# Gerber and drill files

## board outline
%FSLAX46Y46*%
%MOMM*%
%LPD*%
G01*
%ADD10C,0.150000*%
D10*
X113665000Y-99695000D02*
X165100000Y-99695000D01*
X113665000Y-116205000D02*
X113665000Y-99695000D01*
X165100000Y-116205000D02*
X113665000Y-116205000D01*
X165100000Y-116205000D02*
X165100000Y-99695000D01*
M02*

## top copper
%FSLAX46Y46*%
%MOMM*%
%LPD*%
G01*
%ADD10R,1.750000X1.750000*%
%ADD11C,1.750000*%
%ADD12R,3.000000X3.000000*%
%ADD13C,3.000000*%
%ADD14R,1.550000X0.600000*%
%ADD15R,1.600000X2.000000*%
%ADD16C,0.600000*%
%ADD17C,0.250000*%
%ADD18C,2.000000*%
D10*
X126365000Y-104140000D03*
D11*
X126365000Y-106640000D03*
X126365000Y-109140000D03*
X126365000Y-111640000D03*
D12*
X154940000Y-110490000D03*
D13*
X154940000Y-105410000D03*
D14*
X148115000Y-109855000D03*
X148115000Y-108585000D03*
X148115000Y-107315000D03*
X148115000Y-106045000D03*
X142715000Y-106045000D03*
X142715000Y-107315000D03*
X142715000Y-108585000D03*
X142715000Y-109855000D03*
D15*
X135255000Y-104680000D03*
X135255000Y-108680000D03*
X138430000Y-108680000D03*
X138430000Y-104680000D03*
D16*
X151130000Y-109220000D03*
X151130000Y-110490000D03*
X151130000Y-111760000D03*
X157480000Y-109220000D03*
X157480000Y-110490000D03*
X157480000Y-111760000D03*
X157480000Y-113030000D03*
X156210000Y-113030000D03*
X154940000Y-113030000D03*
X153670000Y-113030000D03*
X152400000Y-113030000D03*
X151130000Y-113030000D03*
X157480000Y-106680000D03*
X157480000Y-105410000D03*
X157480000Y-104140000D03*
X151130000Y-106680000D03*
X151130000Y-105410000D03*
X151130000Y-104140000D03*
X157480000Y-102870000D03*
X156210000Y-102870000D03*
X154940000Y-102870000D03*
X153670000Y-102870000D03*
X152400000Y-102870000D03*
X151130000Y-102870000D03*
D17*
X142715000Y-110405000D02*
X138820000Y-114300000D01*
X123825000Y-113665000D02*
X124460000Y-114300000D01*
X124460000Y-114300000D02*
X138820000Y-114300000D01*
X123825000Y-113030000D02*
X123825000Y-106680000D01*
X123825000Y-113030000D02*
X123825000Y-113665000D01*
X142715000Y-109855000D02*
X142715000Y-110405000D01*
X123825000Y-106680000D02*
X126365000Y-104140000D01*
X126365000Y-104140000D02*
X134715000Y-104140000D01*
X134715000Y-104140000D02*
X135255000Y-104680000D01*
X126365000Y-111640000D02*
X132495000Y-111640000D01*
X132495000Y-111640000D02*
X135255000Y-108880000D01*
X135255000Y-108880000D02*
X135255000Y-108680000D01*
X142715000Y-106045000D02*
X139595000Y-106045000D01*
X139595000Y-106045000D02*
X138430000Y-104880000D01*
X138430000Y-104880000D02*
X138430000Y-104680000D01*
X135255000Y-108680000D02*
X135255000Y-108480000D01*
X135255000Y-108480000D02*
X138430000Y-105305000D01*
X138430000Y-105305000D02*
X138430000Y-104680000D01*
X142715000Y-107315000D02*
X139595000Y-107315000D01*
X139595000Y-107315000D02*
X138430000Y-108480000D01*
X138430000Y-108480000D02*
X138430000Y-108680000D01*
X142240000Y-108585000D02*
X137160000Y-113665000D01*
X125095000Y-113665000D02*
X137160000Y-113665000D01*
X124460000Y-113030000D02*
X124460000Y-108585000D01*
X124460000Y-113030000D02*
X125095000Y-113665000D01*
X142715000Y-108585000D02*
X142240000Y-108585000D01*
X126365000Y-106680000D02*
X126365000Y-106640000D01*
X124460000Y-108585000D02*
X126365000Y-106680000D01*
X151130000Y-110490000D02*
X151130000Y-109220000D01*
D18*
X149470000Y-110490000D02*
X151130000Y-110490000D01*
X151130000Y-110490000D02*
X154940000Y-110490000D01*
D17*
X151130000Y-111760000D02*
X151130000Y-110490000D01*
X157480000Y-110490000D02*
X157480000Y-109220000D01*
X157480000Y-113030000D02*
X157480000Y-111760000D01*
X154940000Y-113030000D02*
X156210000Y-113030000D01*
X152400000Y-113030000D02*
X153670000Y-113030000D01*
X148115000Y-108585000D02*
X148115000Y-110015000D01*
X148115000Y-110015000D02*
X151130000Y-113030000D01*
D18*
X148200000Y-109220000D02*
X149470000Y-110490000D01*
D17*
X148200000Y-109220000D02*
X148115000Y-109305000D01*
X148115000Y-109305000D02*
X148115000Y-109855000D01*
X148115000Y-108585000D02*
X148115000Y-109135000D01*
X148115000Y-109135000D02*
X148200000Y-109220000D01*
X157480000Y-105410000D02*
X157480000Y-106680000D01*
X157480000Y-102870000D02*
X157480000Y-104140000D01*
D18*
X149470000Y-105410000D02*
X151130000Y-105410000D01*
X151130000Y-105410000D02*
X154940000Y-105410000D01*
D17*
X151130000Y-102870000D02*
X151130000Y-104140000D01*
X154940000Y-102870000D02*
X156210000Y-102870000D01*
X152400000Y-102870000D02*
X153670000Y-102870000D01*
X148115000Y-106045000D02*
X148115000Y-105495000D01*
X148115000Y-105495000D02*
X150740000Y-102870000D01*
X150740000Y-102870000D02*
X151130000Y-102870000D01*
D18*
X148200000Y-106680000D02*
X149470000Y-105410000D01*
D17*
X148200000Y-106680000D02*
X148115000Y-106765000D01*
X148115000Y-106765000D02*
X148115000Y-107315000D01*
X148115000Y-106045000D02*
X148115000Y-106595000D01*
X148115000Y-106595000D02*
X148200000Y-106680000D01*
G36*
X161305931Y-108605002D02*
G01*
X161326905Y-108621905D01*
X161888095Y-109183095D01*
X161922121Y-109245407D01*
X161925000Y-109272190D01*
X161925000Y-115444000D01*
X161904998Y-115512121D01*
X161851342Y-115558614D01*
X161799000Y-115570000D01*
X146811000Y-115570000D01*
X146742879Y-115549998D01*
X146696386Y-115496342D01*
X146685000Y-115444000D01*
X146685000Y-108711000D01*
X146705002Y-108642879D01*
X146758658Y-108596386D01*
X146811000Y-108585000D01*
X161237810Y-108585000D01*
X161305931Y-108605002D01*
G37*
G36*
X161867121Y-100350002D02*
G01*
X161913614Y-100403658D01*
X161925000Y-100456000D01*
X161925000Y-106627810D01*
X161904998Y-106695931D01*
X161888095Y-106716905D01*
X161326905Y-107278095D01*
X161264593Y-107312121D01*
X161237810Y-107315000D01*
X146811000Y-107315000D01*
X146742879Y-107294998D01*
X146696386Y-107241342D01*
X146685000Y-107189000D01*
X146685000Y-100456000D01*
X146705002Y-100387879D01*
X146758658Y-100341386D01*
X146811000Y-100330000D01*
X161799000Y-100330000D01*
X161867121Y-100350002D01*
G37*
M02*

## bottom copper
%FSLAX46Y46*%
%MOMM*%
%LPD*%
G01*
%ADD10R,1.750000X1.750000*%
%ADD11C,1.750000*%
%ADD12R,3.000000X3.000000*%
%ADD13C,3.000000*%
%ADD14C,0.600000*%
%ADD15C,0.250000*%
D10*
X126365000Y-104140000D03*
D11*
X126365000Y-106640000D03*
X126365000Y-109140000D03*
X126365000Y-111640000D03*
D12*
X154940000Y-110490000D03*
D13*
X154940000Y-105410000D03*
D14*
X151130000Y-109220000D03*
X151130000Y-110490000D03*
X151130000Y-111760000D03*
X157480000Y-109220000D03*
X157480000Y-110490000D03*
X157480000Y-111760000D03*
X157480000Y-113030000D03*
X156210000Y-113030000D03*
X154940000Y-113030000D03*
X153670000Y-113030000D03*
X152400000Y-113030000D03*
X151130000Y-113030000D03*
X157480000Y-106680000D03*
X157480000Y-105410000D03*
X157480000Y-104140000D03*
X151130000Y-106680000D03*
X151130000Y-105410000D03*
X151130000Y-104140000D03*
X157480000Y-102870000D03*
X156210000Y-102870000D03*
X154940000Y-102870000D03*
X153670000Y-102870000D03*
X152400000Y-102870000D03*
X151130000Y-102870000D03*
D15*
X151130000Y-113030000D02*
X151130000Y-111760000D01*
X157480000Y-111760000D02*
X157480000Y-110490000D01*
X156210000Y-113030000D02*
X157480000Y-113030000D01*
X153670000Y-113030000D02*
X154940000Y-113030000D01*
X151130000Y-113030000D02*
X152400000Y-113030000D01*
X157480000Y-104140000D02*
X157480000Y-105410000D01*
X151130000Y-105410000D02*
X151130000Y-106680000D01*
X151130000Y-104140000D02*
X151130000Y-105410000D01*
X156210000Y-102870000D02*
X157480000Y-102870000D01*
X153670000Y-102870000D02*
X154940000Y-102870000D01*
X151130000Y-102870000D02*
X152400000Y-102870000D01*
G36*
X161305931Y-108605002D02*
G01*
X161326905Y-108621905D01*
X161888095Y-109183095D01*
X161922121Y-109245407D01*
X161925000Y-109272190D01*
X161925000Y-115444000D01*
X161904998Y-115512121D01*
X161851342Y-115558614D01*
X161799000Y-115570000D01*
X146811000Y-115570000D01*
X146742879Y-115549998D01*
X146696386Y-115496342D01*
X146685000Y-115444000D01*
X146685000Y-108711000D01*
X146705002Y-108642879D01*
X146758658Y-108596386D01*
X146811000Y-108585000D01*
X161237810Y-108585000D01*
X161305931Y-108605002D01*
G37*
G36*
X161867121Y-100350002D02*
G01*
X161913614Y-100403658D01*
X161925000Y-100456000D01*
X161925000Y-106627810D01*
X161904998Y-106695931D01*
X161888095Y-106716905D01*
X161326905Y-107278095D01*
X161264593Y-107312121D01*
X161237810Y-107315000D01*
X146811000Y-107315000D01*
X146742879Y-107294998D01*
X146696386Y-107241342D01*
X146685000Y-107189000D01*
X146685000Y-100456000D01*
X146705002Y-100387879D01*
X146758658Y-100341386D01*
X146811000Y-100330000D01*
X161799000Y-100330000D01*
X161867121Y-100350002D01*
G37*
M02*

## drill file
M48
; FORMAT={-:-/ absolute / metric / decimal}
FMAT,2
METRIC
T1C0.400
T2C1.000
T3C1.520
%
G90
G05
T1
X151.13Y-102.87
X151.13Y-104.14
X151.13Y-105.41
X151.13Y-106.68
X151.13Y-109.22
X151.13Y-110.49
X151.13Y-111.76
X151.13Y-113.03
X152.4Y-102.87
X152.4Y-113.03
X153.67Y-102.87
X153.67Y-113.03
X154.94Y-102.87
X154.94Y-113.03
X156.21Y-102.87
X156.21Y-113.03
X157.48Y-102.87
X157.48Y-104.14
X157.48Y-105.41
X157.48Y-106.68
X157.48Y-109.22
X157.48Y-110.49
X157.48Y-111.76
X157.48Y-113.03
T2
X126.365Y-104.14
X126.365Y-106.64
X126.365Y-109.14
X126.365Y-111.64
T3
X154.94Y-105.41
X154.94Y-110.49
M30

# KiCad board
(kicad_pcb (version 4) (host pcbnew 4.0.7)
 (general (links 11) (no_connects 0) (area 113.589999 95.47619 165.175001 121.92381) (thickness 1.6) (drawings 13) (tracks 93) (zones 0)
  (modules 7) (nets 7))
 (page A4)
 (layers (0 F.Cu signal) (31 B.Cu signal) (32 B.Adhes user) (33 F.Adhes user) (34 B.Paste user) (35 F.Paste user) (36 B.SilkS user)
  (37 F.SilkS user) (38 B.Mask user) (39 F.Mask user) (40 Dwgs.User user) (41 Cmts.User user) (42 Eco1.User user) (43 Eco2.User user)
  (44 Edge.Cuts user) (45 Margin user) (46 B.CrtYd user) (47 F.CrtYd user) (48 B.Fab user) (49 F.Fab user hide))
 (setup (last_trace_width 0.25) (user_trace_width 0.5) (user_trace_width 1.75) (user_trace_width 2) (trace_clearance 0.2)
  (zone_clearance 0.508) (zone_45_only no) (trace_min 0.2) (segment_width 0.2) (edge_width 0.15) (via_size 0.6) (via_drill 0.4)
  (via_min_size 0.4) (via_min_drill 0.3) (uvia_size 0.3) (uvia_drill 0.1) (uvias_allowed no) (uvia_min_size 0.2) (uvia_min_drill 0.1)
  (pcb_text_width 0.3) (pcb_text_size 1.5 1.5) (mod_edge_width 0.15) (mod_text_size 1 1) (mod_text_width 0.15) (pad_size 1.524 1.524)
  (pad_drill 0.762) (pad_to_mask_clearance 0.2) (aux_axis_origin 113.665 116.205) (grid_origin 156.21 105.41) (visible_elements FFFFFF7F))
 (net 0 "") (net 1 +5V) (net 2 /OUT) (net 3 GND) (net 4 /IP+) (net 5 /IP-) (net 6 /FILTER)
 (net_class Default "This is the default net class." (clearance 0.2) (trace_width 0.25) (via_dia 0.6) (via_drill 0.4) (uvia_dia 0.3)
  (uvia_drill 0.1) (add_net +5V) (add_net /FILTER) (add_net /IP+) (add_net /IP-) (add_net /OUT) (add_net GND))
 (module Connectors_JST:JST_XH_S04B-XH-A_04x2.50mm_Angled (layer F.Cu) (at 126.365 104.14 270)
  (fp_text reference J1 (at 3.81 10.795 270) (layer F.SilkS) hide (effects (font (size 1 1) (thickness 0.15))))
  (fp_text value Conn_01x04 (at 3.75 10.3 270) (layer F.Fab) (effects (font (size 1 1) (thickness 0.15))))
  (pad 1 thru_hole rect (at 0 0 270) (size 1.75 1.75) (drill 1) (layers *.Cu *.Mask F.SilkS) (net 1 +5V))
  (pad 2 thru_hole circle (at 2.5 0 270) (size 1.75 1.75) (drill 1) (layers *.Cu *.Mask F.SilkS) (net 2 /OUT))
  (pad 3 thru_hole circle (at 5 0 270) (size 1.75 1.75) (drill 1) (layers *.Cu *.Mask F.SilkS))
  (pad 4 thru_hole circle (at 7.5 0 270) (size 1.75 1.75) (drill 1) (layers *.Cu *.Mask F.SilkS) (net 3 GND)))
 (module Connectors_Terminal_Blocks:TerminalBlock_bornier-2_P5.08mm (layer F.Cu) (at 154.94 110.49 90)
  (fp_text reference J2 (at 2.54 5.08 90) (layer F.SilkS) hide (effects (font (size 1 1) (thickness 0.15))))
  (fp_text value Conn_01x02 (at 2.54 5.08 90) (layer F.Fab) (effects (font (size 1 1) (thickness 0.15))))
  (pad 1 thru_hole rect (at 0 0 90) (size 3 3) (drill 1.52) (layers *.Cu *.Mask) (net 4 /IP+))
  (pad 2 thru_hole circle (at 5.08 0 90) (size 3 3) (drill 1.52) (layers *.Cu *.Mask) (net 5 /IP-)))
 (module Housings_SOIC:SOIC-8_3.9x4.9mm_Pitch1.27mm (layer F.Cu) (at 145.415 107.95 180)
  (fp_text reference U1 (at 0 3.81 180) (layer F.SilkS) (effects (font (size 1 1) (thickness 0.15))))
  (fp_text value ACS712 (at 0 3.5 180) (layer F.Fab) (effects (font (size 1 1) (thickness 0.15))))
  (pad 1 smd rect (at -2.7 -1.905 180) (size 1.55 0.6) (layers F.Cu F.Paste F.Mask) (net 4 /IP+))
  (pad 2 smd rect (at -2.7 -0.635 180) (size 1.55 0.6) (layers F.Cu F.Paste F.Mask) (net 4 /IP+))
  (pad 3 smd rect (at -2.7 0.635 180) (size 1.55 0.6) (layers F.Cu F.Paste F.Mask) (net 5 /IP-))
  (pad 4 smd rect (at -2.7 1.905 180) (size 1.55 0.6) (layers F.Cu F.Paste F.Mask) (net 5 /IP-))
  (pad 5 smd rect (at 2.7 1.905 180) (size 1.55 0.6) (layers F.Cu F.Paste F.Mask) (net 3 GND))
  (pad 6 smd rect (at 2.7 0.635 180) (size 1.55 0.6) (layers F.Cu F.Paste F.Mask) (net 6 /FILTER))
  (pad 7 smd rect (at 2.7 -0.635 180) (size 1.55 0.6) (layers F.Cu F.Paste F.Mask) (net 2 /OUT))
  (pad 8 smd rect (at 2.7 -1.905 180) (size 1.55 0.6) (layers F.Cu F.Paste F.Mask) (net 1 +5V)))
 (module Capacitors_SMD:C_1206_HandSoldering (layer F.Cu) (at 135.255 106.68 270)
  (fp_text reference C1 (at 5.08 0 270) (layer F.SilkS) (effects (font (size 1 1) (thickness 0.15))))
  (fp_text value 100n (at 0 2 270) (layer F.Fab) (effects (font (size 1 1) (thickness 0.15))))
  (pad 1 smd rect (at -2 0 270) (size 2 1.6) (layers F.Cu F.Paste F.Mask) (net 1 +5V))
  (pad 2 smd rect (at 2 0 270) (size 2 1.6) (layers F.Cu F.Paste F.Mask) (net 3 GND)))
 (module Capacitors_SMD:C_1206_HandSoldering (layer F.Cu) (at 138.43 106.68 90)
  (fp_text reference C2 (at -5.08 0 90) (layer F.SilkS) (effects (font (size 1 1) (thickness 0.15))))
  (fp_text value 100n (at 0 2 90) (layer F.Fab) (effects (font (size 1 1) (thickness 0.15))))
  (pad 1 smd rect (at -2 0 90) (size 2 1.6) (layers F.Cu F.Paste F.Mask) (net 6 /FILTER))
  (pad 2 smd rect (at 2 0 90) (size 2 1.6) (layers F.Cu F.Paste F.Mask) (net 3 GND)))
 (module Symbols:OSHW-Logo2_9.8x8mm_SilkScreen (layer B.Cu) (at 120.015 107.95 270)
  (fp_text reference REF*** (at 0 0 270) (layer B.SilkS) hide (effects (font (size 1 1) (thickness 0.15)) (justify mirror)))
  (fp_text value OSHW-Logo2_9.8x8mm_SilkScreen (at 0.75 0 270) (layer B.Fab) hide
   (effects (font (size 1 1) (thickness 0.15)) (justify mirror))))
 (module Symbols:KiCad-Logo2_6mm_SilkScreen (layer B.Cu) (at 160.655 107.95 270)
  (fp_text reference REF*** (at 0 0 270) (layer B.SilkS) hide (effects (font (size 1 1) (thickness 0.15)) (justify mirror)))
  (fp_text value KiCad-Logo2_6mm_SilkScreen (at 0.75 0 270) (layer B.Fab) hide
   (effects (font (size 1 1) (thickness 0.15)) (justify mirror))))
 (gr_line (start 113.665 99.695) (end 165.1 99.695) (layer Edge.Cuts) (width 0.15))
 (gr_line (start 113.665 116.205) (end 113.665 99.695) (layer Edge.Cuts) (width 0.15))
 (gr_line (start 165.1 116.205) (end 113.665 116.205) (layer Edge.Cuts) (width 0.15))
 (gr_line (start 165.1 116.205) (end 165.1 99.695) (layer Edge.Cuts) (width 0.15))
 (segment (start 142.715 110.405) (end 138.82 114.3) (width 0.25) (layer F.Cu) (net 1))
 (segment (start 123.825 113.665) (end 124.46 114.3) (width 0.25) (layer F.Cu) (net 1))
 (segment (start 124.46 114.3) (end 138.82 114.3) (width 0.25) (layer F.Cu) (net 1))
 (segment (start 123.825 113.03) (end 123.825 106.68) (width 0.25) (layer F.Cu) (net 1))
 (segment (start 123.825 113.03) (end 123.825 113.665) (width 0.25) (layer F.Cu) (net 1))
 (segment (start 142.715 109.855) (end 142.715 110.405) (width 0.25) (layer F.Cu) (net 1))
 (segment (start 123.825 106.68) (end 126.365 104.14) (width 0.25) (layer F.Cu) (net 1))
 (segment (start 126.365 104.14) (end 134.715 104.14) (width 0.25) (layer F.Cu) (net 1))
 (segment (start 134.715 104.14) (end 135.255 104.68) (width 0.25) (layer F.Cu) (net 1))
 (segment (start 126.365 111.64) (end 132.495 111.64) (width 0.25) (layer F.Cu) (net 3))
 (segment (start 132.495 111.64) (end 135.255 108.88) (width 0.25) (layer F.Cu) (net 3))
 (segment (start 135.255 108.88) (end 135.255 108.68) (width 0.25) (layer F.Cu) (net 3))
 (segment (start 142.715 106.045) (end 139.595 106.045) (width 0.25) (layer F.Cu) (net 3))
 (segment (start 139.595 106.045) (end 138.43 104.88) (width 0.25) (layer F.Cu) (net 3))
 (segment (start 138.43 104.88) (end 138.43 104.68) (width 0.25) (layer F.Cu) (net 3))
 (segment (start 135.255 108.68) (end 135.255 108.48) (width 0.25) (layer F.Cu) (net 3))
 (segment (start 135.255 108.48) (end 138.43 105.305) (width 0.25) (layer F.Cu) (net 3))
 (segment (start 138.43 105.305) (end 138.43 104.68) (width 0.25) (layer F.Cu) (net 3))
 (segment (start 142.715 107.315) (end 139.595 107.315) (width 0.25) (layer F.Cu) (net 6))
 (segment (start 139.595 107.315) (end 138.43 108.48) (width 0.25) (layer F.Cu) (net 6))
 (segment (start 138.43 108.48) (end 138.43 108.68) (width 0.25) (layer F.Cu) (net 6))
 (segment (start 142.24 108.585) (end 137.16 113.665) (width 0.25) (layer F.Cu) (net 2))
 (segment (start 125.095 113.665) (end 137.16 113.665) (width 0.25) (layer F.Cu) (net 2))
 (segment (start 124.46 113.03) (end 124.46 108.585) (width 0.25) (layer F.Cu) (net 2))
 (segment (start 124.46 113.03) (end 125.095 113.665) (width 0.25) (layer F.Cu) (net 2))
 (segment (start 142.715 108.585) (end 142.24 108.585) (width 0.25) (layer F.Cu) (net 2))
 (segment (start 126.365 106.68) (end 126.365 106.64) (width 0.25) (layer F.Cu) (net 2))
 (segment (start 124.46 108.585) (end 126.365 106.68) (width 0.25) (layer F.Cu) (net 2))
 (segment (start 151.13 110.49) (end 151.13 109.22) (width 0.25) (layer F.Cu) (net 4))
 (via (at 151.13 109.22) (size 0.6) (drill 0.4) (layers F.Cu B.Cu) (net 4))
 (segment (start 149.47 110.49) (end 151.13 110.49) (width 2) (layer F.Cu) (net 4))
 (segment (start 151.13 110.49) (end 154.94 110.49) (width 2) (layer F.Cu) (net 4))
 (segment (start 151.13 111.76) (end 151.13 110.49) (width 0.25) (layer F.Cu) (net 4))
 (via (at 151.13 110.49) (size 0.6) (drill 0.4) (layers F.Cu B.Cu) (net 4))
 (segment (start 151.13 113.03) (end 151.13 111.76) (width 0.25) (layer B.Cu) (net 4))
 (via (at 151.13 111.76) (size 0.6) (drill 0.4) (layers F.Cu B.Cu) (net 4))
 (segment (start 157.48 110.49) (end 157.48 109.22) (width 0.25) (layer F.Cu) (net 4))
 (via (at 157.48 109.22) (size 0.6) (drill 0.4) (layers F.Cu B.Cu) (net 4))
 (segment (start 157.48 111.76) (end 157.48 110.49) (width 0.25) (layer B.Cu) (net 4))
 (via (at 157.48 110.49) (size 0.6) (drill 0.4) (layers F.Cu B.Cu) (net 4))
 (segment (start 157.48 113.03) (end 157.48 111.76) (width 0.25) (layer F.Cu) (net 4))
 (via (at 157.48 111.76) (size 0.6) (drill 0.4) (layers F.Cu B.Cu) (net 4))
 (segment (start 156.21 113.03) (end 157.48 113.03) (width 0.25) (layer B.Cu) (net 4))
 (via (at 157.48 113.03) (size 0.6) (drill 0.4) (layers F.Cu B.Cu) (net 4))
 (segment (start 154.94 113.03) (end 156.21 113.03) (width 0.25) (layer F.Cu) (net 4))
 (via (at 156.21 113.03) (size 0.6) (drill 0.4) (layers F.Cu B.Cu) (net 4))
 (segment (start 153.67 113.03) (end 154.94 113.03) (width 0.25) (layer B.Cu) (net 4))
 (via (at 154.94 113.03) (size 0.6) (drill 0.4) (layers F.Cu B.Cu) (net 4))
 (segment (start 152.4 113.03) (end 153.67 113.03) (width 0.25) (layer F.Cu) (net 4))
 (via (at 153.67 113.03) (size 0.6) (drill 0.4) (layers F.Cu B.Cu) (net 4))
 (segment (start 151.13 113.03) (end 152.4 113.03) (width 0.25) (layer B.Cu) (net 4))
 (via (at 152.4 113.03) (size 0.6) (drill 0.4) (layers F.Cu B.Cu) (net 4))
 (segment (start 148.115 108.585) (end 148.115 110.015) (width 0.25) (layer F.Cu) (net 4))
 (segment (start 148.115 110.015) (end 151.13 113.03) (width 0.25) (layer F.Cu) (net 4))
 (via (at 151.13 113.03) (size 0.6) (drill 0.4) (layers F.Cu B.Cu) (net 4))
 (segment (start 148.2 109.22) (end 149.47 110.49) (width 2) (layer F.Cu) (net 4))
 (segment (start 148.2 109.22) (end 148.115 109.305) (width 0.25) (layer F.Cu) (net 4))
 (segment (start 148.115 109.305) (end 148.115 109.855) (width 0.25) (layer F.Cu) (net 4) (status 20))
 (segment (start 148.115 108.585) (end 148.115 109.135) (width 0.25) (layer F.Cu) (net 4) (status 10))
 (segment (start 148.115 109.135) (end 148.2 109.22) (width 0.25) (layer F.Cu) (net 4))
 (segment (start 157.48 105.41) (end 157.48 106.68) (width 0.25) (layer F.Cu) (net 5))
 (via (at 157.48 106.68) (size 0.6) (drill 0.4) (layers F.Cu B.Cu) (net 5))
 (segment (start 157.48 104.14) (end 157.48 105.41) (width 0.25) (layer B.Cu) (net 5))
 (via (at 157.48 105.41) (size 0.6) (drill 0.4) (layers F.Cu B.Cu) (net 5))
 (segment (start 157.48 102.87) (end 157.48 104.14) (width 0.25) (layer F.Cu) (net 5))
 (via (at 157.48 104.14) (size 0.6) (drill 0.4) (layers F.Cu B.Cu) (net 5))
 (segment (start 151.13 105.41) (end 151.13 106.68) (width 0.25) (layer B.Cu) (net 5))
 (via (at 151.13 106.68) (size 0.6) (drill 0.4) (layers F.Cu B.Cu) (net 5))
 (segment (start 149.47 105.41) (end 151.13 105.41) (width 2) (layer F.Cu) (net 5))
 (segment (start 151.13 105.41) (end 154.94 105.41) (width 2) (layer F.Cu) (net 5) (status 20))
 (segment (start 151.13 104.14) (end 151.13 105.41) (width 0.25) (layer B.Cu) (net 5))
 (via (at 151.13 105.41) (size 0.6) (drill 0.4) (layers F.Cu B.Cu) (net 5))
 (segment (start 151.13 102.87) (end 151.13 104.14) (width 0.25) (layer F.Cu) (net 5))
 (via (at 151.13 104.14) (size 0.6) (drill 0.4) (layers F.Cu B.Cu) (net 5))
 (segment (start 156.21 102.87) (end 157.48 102.87) (width 0.25) (layer B.Cu) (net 5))
 (via (at 157.48 102.87) (size 0.6) (drill 0.4) (layers F.Cu B.Cu) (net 5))
 (segment (start 154.94 102.87) (end 156.21 102.87) (width 0.25) (layer F.Cu) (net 5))
 (via (at 156.21 102.87) (size 0.6) (drill 0.4) (layers F.Cu B.Cu) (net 5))
 (segment (start 153.67 102.87) (end 154.94 102.87) (width 0.25) (layer B.Cu) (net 5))
 (via (at 154.94 102.87) (size 0.6) (drill 0.4) (layers F.Cu B.Cu) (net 5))
 (segment (start 152.4 102.87) (end 153.67 102.87) (width 0.25) (layer F.Cu) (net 5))
 (via (at 153.67 102.87) (size 0.6) (drill 0.4) (layers F.Cu B.Cu) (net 5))
 (segment (start 151.13 102.87) (end 152.4 102.87) (width 0.25) (layer B.Cu) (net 5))
 (via (at 152.4 102.87) (size 0.6) (drill 0.4) (layers F.Cu B.Cu) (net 5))
 (segment (start 148.115 106.045) (end 148.115 105.495) (width 0.25) (layer F.Cu) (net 5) (status 10))
 (segment (start 148.115 105.495) (end 150.74 102.87) (width 0.25) (layer F.Cu) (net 5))
 (segment (start 150.74 102.87) (end 151.13 102.87) (width 0.25) (layer F.Cu) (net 5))
 (via (at 151.13 102.87) (size 0.6) (drill 0.4) (layers F.Cu B.Cu) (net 5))
 (segment (start 148.2 106.68) (end 149.47 105.41) (width 2) (layer F.Cu) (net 5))
 (segment (start 148.2 106.68) (end 148.115 106.765) (width 0.25) (layer F.Cu) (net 5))
 (segment (start 148.115 106.765) (end 148.115 107.315) (width 0.25) (layer F.Cu) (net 5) (status 20))
 (segment (start 148.115 106.045) (end 148.115 106.595) (width 0.25) (layer F.Cu) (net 5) (status 10))
 (segment (start 148.115 106.595) (end 148.2 106.68) (width 0.25) (layer F.Cu) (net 5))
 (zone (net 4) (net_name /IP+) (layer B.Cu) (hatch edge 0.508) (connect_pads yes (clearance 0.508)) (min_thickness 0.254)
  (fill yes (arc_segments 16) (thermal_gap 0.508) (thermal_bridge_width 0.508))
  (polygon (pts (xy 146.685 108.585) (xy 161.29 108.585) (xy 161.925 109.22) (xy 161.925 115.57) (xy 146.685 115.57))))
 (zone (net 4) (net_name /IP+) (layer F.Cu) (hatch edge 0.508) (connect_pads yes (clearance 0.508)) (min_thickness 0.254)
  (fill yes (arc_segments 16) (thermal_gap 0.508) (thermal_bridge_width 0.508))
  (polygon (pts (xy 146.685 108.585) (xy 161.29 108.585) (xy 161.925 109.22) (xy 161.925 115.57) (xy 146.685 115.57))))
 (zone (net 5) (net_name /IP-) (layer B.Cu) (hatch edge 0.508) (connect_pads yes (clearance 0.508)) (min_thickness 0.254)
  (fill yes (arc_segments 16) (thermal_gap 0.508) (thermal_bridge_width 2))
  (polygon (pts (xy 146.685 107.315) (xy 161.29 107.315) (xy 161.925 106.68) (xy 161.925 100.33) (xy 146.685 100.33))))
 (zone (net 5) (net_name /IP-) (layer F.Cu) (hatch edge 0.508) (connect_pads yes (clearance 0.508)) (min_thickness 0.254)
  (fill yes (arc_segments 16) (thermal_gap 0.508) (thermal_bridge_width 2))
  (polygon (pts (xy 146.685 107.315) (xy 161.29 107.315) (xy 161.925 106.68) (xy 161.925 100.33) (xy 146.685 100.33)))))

